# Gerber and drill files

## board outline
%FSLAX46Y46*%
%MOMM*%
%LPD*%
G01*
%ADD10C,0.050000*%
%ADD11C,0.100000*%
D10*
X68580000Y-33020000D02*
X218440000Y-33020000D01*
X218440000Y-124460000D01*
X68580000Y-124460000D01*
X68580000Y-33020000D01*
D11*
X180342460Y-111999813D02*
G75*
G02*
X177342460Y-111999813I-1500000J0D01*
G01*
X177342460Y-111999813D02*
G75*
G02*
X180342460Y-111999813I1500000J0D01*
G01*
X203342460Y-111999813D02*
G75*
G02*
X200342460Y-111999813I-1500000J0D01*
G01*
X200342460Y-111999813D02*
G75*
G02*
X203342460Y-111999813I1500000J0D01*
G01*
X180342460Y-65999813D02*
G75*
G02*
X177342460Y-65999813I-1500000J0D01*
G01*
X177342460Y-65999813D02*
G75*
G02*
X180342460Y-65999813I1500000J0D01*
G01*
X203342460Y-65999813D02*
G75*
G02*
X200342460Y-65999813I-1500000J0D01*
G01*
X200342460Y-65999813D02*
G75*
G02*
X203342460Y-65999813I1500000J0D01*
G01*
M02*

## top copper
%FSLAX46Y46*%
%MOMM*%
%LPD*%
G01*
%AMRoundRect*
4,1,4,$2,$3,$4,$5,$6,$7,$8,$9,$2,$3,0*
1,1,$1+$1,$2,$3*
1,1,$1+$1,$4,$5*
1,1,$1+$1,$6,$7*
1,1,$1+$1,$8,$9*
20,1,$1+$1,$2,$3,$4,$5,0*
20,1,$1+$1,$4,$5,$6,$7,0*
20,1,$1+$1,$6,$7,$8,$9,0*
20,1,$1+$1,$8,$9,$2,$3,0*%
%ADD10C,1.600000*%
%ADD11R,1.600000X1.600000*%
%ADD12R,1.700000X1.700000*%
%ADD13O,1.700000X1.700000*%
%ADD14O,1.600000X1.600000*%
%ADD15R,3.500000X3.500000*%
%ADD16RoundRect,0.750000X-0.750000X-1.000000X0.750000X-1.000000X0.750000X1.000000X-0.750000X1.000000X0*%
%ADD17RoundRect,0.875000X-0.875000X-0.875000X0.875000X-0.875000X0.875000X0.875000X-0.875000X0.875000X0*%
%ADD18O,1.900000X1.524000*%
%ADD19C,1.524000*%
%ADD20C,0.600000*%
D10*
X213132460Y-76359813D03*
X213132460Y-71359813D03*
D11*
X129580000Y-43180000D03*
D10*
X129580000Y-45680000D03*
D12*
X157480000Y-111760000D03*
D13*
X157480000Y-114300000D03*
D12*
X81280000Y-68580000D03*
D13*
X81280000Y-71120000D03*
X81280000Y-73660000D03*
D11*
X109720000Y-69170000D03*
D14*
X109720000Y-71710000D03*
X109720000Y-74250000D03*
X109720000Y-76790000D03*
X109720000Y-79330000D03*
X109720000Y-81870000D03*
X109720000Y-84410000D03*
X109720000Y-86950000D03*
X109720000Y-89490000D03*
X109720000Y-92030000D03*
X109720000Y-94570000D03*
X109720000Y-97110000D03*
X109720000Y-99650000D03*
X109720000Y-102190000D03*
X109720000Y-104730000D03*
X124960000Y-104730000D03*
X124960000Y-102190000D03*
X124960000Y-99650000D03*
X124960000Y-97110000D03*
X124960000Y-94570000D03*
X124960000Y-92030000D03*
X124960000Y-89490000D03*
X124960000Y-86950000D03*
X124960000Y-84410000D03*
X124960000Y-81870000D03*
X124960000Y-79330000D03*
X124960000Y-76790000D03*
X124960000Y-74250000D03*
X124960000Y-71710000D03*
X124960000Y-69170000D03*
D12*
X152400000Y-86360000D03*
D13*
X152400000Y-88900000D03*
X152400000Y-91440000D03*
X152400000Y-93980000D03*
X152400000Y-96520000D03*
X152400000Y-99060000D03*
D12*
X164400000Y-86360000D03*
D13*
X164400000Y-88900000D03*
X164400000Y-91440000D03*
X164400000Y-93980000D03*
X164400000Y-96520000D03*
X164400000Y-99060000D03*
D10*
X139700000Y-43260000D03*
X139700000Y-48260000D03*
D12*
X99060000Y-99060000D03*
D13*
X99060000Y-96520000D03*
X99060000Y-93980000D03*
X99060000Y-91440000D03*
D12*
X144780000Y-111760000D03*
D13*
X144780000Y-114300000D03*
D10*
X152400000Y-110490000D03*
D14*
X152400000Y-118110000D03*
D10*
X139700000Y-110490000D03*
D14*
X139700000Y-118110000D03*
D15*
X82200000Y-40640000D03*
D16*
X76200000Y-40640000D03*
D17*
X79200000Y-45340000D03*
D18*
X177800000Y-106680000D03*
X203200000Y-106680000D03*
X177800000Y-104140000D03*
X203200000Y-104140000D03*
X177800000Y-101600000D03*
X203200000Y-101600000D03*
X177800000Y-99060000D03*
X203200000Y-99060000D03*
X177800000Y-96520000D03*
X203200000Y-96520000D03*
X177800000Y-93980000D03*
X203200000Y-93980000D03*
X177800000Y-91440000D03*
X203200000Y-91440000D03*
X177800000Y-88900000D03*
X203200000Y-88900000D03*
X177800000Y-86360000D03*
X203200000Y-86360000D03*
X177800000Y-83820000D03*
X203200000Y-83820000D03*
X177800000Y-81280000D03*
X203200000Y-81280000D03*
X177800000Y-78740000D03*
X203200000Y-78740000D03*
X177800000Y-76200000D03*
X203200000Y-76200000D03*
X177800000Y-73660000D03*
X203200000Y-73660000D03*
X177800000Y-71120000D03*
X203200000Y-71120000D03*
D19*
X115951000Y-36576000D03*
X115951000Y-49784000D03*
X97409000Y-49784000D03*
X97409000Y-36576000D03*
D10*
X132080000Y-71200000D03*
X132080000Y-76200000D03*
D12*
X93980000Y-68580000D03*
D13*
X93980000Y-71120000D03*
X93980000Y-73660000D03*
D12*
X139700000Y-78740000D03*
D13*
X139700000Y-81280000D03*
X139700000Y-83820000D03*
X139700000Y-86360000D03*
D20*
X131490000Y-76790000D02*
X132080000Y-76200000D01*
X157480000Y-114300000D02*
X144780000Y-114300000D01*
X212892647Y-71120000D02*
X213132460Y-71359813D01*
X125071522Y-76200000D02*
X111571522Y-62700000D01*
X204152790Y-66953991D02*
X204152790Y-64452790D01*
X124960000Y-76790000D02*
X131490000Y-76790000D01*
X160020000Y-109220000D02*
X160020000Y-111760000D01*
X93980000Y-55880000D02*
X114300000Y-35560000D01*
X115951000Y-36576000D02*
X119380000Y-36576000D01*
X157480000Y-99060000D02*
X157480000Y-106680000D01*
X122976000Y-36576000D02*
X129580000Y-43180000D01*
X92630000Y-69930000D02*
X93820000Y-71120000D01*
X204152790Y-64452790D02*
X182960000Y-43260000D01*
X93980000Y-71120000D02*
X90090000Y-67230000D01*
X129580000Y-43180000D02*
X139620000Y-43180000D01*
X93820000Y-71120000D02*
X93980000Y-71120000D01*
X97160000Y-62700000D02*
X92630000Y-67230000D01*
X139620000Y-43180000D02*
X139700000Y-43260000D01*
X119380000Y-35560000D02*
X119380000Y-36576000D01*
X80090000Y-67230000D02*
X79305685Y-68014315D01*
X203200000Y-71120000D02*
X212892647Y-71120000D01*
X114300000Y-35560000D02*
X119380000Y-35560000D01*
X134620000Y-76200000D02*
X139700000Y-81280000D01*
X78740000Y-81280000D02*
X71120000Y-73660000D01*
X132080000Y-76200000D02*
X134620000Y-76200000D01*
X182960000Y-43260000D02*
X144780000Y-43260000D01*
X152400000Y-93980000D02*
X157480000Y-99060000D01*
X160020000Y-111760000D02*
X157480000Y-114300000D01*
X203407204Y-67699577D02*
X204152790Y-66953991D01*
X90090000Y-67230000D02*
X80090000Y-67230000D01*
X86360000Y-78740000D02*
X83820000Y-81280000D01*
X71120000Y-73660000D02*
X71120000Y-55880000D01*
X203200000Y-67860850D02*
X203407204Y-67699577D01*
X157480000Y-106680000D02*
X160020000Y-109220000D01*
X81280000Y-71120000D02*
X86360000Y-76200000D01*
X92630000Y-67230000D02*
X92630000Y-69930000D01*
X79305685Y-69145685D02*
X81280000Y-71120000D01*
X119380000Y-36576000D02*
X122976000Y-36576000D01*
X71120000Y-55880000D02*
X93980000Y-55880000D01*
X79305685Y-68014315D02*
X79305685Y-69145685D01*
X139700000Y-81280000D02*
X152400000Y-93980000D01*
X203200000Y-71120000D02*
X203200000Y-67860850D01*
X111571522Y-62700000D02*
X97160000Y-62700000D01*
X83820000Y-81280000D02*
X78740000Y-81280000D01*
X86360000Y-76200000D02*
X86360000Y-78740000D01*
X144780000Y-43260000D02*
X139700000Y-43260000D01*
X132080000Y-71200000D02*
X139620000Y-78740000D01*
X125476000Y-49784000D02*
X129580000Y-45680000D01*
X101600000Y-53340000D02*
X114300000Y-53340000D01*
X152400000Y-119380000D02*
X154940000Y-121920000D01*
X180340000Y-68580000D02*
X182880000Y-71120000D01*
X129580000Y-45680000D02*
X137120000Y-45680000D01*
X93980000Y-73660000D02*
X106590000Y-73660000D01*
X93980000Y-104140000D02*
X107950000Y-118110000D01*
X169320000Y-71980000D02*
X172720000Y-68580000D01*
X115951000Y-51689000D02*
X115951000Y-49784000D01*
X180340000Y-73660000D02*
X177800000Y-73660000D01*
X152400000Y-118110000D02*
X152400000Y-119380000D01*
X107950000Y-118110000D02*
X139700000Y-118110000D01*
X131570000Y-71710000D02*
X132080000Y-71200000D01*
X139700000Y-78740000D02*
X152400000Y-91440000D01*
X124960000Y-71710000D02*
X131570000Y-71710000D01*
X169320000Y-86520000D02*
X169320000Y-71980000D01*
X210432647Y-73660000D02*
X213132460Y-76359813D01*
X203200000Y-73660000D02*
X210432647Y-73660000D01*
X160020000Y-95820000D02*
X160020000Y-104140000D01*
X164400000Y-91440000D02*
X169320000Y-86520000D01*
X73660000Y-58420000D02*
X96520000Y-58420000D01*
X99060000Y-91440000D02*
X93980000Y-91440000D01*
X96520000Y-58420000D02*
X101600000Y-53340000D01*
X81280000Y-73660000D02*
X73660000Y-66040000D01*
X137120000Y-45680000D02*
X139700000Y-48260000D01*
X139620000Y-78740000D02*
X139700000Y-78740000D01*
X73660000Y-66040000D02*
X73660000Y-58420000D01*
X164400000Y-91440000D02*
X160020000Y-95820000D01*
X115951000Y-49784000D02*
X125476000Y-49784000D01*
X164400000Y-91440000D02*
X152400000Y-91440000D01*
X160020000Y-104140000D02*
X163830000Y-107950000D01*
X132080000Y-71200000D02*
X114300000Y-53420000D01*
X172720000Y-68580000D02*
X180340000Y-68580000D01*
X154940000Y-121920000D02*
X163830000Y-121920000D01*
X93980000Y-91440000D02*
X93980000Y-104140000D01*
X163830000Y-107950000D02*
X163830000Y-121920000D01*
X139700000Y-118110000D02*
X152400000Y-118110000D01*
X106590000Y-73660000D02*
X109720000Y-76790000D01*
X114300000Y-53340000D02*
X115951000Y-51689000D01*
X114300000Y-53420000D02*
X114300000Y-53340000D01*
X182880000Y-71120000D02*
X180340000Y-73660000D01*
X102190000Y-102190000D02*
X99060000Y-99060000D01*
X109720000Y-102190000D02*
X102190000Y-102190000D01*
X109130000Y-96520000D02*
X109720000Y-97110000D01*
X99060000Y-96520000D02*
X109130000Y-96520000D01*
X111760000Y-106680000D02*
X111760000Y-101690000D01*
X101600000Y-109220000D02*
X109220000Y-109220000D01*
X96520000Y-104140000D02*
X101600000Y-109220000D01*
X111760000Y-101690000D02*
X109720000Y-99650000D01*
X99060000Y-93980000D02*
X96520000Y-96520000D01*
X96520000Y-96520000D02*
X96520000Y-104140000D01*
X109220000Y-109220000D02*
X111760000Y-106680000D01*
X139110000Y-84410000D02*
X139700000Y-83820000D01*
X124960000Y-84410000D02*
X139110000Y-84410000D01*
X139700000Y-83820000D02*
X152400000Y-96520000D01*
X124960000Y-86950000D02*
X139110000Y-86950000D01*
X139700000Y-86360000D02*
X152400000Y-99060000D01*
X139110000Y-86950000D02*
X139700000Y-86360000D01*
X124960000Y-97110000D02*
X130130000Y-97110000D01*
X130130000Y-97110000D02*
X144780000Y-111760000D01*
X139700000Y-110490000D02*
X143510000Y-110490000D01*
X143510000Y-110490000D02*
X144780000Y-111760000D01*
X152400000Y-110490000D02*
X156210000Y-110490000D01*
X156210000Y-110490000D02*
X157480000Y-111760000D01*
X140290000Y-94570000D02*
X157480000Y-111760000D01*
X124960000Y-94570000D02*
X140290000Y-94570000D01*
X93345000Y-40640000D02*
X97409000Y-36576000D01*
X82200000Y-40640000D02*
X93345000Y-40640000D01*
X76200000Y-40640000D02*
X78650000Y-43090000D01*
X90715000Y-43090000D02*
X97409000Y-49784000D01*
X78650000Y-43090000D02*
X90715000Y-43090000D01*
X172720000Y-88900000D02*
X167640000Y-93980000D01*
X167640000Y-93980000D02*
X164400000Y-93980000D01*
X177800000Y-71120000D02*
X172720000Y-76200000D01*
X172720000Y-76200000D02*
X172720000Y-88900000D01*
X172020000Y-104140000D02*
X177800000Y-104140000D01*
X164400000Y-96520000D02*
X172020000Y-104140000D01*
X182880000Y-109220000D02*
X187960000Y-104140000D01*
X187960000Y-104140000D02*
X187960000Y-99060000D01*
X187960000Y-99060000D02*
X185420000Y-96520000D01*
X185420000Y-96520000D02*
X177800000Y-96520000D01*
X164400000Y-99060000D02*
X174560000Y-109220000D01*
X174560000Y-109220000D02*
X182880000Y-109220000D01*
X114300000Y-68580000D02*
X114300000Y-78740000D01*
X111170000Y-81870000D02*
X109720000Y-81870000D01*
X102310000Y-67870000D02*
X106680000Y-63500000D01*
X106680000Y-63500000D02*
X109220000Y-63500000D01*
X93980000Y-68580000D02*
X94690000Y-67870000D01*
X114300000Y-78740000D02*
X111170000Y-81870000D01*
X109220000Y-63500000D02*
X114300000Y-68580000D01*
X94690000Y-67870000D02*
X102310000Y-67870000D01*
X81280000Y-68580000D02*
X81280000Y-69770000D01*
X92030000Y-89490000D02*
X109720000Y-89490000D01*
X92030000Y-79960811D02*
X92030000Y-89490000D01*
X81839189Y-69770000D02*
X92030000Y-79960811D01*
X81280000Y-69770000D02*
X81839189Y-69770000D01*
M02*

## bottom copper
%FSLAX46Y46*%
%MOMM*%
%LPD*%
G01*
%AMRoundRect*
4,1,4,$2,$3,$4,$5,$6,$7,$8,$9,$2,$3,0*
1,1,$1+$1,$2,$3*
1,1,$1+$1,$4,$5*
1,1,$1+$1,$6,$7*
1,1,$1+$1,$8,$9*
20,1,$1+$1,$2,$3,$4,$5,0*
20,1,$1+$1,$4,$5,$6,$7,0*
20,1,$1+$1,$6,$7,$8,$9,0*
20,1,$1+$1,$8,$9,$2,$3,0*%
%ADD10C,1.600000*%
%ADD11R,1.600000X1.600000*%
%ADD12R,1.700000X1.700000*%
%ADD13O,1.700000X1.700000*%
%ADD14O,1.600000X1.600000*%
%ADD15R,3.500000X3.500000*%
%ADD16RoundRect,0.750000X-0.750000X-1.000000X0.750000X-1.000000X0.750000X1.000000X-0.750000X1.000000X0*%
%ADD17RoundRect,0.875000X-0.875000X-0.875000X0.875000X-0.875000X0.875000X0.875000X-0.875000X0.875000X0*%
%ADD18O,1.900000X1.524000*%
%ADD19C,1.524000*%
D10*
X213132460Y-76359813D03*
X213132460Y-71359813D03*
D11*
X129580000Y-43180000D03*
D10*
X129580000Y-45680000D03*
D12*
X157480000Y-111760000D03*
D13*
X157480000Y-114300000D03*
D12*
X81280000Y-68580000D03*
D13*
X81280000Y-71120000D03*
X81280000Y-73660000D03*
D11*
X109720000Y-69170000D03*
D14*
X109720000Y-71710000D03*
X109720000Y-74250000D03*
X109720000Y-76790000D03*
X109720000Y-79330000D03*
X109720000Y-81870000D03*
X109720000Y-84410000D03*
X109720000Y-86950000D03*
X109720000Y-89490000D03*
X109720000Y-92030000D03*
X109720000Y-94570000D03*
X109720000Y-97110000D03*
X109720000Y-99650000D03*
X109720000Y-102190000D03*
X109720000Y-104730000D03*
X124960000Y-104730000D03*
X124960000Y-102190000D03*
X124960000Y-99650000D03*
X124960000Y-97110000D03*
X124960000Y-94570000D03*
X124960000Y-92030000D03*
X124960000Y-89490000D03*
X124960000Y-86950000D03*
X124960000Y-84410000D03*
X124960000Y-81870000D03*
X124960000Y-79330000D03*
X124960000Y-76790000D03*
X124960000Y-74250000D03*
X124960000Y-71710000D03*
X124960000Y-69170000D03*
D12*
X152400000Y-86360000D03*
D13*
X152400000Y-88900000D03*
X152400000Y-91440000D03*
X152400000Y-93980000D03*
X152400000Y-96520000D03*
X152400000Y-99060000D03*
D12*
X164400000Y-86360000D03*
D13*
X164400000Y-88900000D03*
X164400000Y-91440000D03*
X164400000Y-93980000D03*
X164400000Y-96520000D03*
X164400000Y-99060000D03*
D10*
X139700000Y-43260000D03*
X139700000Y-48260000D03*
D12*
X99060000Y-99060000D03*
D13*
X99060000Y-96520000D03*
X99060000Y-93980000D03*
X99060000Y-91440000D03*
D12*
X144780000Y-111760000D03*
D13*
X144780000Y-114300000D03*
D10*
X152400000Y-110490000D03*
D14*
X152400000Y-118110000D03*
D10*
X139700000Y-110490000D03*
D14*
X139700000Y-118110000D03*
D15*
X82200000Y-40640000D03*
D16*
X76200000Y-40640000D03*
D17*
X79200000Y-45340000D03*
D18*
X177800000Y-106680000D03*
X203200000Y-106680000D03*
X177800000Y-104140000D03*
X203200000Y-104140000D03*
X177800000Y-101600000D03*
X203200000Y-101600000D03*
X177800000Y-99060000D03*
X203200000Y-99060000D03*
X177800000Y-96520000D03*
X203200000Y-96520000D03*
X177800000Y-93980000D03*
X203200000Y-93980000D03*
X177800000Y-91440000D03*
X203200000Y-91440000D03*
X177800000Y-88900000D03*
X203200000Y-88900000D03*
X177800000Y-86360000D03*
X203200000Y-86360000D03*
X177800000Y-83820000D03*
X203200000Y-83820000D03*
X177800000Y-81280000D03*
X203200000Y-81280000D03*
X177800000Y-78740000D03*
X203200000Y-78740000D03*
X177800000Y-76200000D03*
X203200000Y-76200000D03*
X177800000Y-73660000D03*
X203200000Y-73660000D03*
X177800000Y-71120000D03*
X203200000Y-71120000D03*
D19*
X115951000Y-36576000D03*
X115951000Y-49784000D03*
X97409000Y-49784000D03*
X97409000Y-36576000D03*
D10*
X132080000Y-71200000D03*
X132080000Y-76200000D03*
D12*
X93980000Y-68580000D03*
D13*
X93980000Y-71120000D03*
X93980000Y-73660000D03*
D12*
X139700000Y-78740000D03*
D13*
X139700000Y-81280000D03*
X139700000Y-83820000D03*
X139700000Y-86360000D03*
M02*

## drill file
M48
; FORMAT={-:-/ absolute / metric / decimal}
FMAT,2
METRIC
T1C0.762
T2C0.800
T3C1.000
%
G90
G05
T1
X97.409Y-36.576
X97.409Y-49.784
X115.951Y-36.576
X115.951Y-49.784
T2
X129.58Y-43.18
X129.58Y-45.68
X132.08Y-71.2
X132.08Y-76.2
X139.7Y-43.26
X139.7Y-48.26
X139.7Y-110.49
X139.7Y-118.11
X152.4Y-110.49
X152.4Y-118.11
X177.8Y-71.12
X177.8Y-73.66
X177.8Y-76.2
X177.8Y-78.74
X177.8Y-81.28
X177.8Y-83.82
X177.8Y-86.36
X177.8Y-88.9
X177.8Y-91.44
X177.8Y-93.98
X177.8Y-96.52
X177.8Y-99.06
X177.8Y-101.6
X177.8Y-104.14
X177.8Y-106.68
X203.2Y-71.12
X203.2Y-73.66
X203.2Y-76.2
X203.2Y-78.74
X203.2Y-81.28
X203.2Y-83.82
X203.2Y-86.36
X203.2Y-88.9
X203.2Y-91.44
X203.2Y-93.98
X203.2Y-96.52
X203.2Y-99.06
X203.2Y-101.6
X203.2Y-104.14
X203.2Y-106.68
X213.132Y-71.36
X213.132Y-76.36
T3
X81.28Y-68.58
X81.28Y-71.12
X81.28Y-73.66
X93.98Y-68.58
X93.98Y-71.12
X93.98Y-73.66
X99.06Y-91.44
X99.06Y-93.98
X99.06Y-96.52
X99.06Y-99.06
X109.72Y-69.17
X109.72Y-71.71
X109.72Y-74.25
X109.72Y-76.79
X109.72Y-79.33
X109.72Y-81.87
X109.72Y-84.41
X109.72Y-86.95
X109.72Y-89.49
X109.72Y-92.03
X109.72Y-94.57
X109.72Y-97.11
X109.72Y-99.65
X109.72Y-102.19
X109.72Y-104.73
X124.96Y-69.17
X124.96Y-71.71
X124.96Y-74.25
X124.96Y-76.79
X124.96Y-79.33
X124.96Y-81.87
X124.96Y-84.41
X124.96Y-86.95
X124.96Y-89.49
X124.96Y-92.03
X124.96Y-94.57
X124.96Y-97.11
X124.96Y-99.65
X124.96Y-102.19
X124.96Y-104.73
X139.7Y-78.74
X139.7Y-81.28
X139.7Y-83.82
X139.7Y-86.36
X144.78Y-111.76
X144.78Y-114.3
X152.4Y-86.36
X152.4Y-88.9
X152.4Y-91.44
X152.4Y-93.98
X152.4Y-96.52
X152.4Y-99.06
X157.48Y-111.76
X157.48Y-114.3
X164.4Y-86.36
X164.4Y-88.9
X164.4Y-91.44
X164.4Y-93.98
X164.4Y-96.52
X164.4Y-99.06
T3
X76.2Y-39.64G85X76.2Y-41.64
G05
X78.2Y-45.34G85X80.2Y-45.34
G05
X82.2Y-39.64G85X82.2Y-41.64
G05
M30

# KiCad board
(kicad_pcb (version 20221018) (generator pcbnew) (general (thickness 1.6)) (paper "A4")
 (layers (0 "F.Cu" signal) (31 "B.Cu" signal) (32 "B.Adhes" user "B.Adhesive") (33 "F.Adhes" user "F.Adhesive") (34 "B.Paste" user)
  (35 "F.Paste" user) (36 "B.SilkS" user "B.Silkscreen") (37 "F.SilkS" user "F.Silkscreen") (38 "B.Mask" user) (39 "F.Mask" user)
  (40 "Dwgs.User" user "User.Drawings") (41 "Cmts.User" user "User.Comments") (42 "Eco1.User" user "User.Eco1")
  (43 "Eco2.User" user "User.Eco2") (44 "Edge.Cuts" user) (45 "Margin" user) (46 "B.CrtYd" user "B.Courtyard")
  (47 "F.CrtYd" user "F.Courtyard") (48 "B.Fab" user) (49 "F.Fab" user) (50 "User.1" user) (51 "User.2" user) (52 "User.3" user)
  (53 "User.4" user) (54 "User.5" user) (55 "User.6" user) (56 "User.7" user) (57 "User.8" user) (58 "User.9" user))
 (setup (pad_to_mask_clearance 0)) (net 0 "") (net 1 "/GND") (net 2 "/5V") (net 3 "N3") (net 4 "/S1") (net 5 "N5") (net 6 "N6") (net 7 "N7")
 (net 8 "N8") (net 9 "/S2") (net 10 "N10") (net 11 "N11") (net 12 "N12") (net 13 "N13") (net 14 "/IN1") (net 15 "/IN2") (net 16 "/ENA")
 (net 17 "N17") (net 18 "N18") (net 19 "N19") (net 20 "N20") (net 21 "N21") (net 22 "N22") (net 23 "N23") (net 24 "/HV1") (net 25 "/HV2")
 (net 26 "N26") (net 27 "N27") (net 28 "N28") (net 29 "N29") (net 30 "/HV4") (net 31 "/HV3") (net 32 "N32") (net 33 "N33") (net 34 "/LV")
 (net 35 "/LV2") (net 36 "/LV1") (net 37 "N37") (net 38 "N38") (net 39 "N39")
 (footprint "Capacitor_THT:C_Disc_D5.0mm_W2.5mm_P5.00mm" (layer "F.Cu") (at 213.13246 76.359813 90)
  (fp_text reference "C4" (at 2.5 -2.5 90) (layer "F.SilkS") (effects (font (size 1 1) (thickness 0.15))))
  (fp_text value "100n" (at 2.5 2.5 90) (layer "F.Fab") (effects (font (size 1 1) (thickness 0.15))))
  (pad "1" thru_hole circle (at 0 0 90) (size 1.6 1.6) (drill 0.8) (layers "*.Cu" "*.Mask") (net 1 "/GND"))
  (pad "2" thru_hole circle (at 5 0 90) (size 1.6 1.6) (drill 0.8) (layers "*.Cu" "*.Mask") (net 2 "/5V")))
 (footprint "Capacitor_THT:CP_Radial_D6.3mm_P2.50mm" (layer "F.Cu") (at 129.58 43.18 -90)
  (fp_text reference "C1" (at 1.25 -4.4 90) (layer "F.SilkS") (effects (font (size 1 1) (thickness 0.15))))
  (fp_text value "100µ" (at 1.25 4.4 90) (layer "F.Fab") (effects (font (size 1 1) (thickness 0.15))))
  (pad "1" thru_hole rect (at 0 0 270) (size 1.6 1.6) (drill 0.8) (layers "*.Cu" "*.Mask") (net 2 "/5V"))
  (pad "2" thru_hole circle (at 2.5 0 270) (size 1.6 1.6) (drill 0.8) (layers "*.Cu" "*.Mask") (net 1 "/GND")))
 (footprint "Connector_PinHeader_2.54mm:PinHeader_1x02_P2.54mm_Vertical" (layer "F.Cu") (at 157.48 111.76)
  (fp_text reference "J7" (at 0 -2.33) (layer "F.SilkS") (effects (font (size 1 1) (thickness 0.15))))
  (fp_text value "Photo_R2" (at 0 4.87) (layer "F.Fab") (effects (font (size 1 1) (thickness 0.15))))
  (pad "1" thru_hole rect (at 0 0) (size 1.7 1.7) (drill 1) (layers "*.Cu" "*.Mask") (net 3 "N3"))
  (pad "2" thru_hole oval (at 0 2.54) (size 1.7 1.7) (drill 1) (layers "*.Cu" "*.Mask") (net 2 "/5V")))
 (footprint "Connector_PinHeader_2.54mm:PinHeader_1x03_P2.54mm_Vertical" (layer "F.Cu") (at 81.28 68.58)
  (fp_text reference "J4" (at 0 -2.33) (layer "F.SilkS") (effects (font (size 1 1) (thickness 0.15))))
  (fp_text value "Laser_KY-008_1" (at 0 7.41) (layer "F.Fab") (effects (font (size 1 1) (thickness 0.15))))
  (pad "1" thru_hole rect (at 0 0) (size 1.7 1.7) (drill 1) (layers "*.Cu" "*.Mask") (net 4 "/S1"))
  (pad "2" thru_hole oval (at 0 2.54) (size 1.7 1.7) (drill 1) (layers "*.Cu" "*.Mask") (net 2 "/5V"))
  (pad "3" thru_hole oval (at 0 5.08) (size 1.7 1.7) (drill 1) (layers "*.Cu" "*.Mask") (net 1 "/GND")))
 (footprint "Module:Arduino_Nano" (layer "F.Cu") (at 109.72 69.17)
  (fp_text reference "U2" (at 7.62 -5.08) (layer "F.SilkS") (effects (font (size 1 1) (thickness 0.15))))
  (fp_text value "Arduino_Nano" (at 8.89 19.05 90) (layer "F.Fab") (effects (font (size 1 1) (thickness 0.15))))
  (pad "1" thru_hole rect (at 0 0) (size 1.6 1.6) (drill 1) (layers "*.Cu" "*.Mask") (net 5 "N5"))
  (pad "2" thru_hole oval (at 0 2.54) (size 1.6 1.6) (drill 1) (layers "*.Cu" "*.Mask") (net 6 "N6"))
  (pad "3" thru_hole oval (at 0 5.08) (size 1.6 1.6) (drill 1) (layers "*.Cu" "*.Mask") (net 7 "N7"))
  (pad "4" thru_hole oval (at 0 7.62) (size 1.6 1.6) (drill 1) (layers "*.Cu" "*.Mask") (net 1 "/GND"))
  (pad "5" thru_hole oval (at 0 10.16) (size 1.6 1.6) (drill 1) (layers "*.Cu" "*.Mask") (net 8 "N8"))
  (pad "6" thru_hole oval (at 0 12.7) (size 1.6 1.6) (drill 1) (layers "*.Cu" "*.Mask") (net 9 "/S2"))
  (pad "7" thru_hole oval (at 0 15.24) (size 1.6 1.6) (drill 1) (layers "*.Cu" "*.Mask") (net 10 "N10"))
  (pad "8" thru_hole oval (at 0 17.78) (size 1.6 1.6) (drill 1) (layers "*.Cu" "*.Mask") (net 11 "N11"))
  (pad "9" thru_hole oval (at 0 20.32) (size 1.6 1.6) (drill 1) (layers "*.Cu" "*.Mask") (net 4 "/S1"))
  (pad "10" thru_hole oval (at 0 22.86) (size 1.6 1.6) (drill 1) (layers "*.Cu" "*.Mask") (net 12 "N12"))
  (pad "11" thru_hole oval (at 0 25.4) (size 1.6 1.6) (drill 1) (layers "*.Cu" "*.Mask") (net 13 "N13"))
  (pad "12" thru_hole oval (at 0 27.94) (size 1.6 1.6) (drill 1) (layers "*.Cu" "*.Mask") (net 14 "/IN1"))
  (pad "13" thru_hole oval (at 0 30.48) (size 1.6 1.6) (drill 1) (layers "*.Cu" "*.Mask") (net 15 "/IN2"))
  (pad "14" thru_hole oval (at 0 33.02) (size 1.6 1.6) (drill 1) (layers "*.Cu" "*.Mask") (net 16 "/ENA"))
  (pad "15" thru_hole oval (at 0 35.56) (size 1.6 1.6) (drill 1) (layers "*.Cu" "*.Mask") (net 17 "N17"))
  (pad "16" thru_hole oval (at 15.24 35.56) (size 1.6 1.6) (drill 1) (layers "*.Cu" "*.Mask") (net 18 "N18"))
  (pad "17" thru_hole oval (at 15.24 33.02) (size 1.6 1.6) (drill 1) (layers "*.Cu" "*.Mask") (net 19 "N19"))
  (pad "18" thru_hole oval (at 15.24 30.48) (size 1.6 1.6) (drill 1) (layers "*.Cu" "*.Mask") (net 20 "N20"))
  (pad "19" thru_hole oval (at 15.24 27.94) (size 1.6 1.6) (drill 1) (layers "*.Cu" "*.Mask") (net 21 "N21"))
  (pad "20" thru_hole oval (at 15.24 25.4) (size 1.6 1.6) (drill 1) (layers "*.Cu" "*.Mask") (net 3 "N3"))
  (pad "21" thru_hole oval (at 15.24 22.86) (size 1.6 1.6) (drill 1) (layers "*.Cu" "*.Mask") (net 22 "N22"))
  (pad "22" thru_hole oval (at 15.24 20.32) (size 1.6 1.6) (drill 1) (layers "*.Cu" "*.Mask") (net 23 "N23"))
  (pad "23" thru_hole oval (at 15.24 17.78) (size 1.6 1.6) (drill 1) (layers "*.Cu" "*.Mask") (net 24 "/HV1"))
  (pad "24" thru_hole oval (at 15.24 15.24) (size 1.6 1.6) (drill 1) (layers "*.Cu" "*.Mask") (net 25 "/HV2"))
  (pad "25" thru_hole oval (at 15.24 12.7) (size 1.6 1.6) (drill 1) (layers "*.Cu" "*.Mask") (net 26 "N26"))
  (pad "26" thru_hole oval (at 15.24 10.16) (size 1.6 1.6) (drill 1) (layers "*.Cu" "*.Mask") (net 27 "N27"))
  (pad "27" thru_hole oval (at 15.24 7.62) (size 1.6 1.6) (drill 1) (layers "*.Cu" "*.Mask") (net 2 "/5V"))
  (pad "28" thru_hole oval (at 15.24 5.08) (size 1.6 1.6) (drill 1) (layers "*.Cu" "*.Mask") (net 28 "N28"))
  (pad "29" thru_hole oval (at 15.24 2.54) (size 1.6 1.6) (drill 1) (layers "*.Cu" "*.Mask") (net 1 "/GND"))
  (pad "30" thru_hole oval (at 15.24 0) (size 1.6 1.6) (drill 1) (layers "*.Cu" "*.Mask") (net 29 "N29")))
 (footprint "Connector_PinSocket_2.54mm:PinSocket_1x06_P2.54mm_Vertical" (layer "F.Cu") (at 152.4 86.36)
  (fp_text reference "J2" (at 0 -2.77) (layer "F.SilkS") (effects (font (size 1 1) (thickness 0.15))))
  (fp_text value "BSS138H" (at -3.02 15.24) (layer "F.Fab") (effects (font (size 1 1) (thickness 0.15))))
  (pad "1" thru_hole rect (at 0 0) (size 1.7 1.7) (drill 1) (layers "*.Cu" "*.Mask") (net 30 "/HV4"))
  (pad "2" thru_hole oval (at 0 2.54) (size 1.7 1.7) (drill 1) (layers "*.Cu" "*.Mask") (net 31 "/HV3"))
  (pad "3" thru_hole oval (at 0 5.08) (size 1.7 1.7) (drill 1) (layers "*.Cu" "*.Mask") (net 1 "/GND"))
  (pad "4" thru_hole oval (at 0 7.62) (size 1.7 1.7) (drill 1) (layers "*.Cu" "*.Mask") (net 2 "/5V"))
  (pad "5" thru_hole oval (at 0 10.16) (size 1.7 1.7) (drill 1) (layers "*.Cu" "*.Mask") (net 25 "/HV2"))
  (pad "6" thru_hole oval (at 0 12.7) (size 1.7 1.7) (drill 1) (layers "*.Cu" "*.Mask") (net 24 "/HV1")))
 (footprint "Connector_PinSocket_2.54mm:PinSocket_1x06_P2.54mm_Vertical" (layer "F.Cu") (at 164.4 86.36)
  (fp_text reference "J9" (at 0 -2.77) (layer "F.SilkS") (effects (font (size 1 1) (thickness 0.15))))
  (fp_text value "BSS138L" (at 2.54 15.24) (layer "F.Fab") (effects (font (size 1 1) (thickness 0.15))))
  (pad "1" thru_hole rect (at 0 0) (size 1.7 1.7) (drill 1) (layers "*.Cu" "*.Mask") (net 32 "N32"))
  (pad "2" thru_hole oval (at 0 2.54) (size 1.7 1.7) (drill 1) (layers "*.Cu" "*.Mask") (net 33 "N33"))
  (pad "3" thru_hole oval (at 0 5.08) (size 1.7 1.7) (drill 1) (layers "*.Cu" "*.Mask") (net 1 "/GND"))
  (pad "4" thru_hole oval (at 0 7.62) (size 1.7 1.7) (drill 1) (layers "*.Cu" "*.Mask") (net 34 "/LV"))
  (pad "5" thru_hole oval (at 0 10.16) (size 1.7 1.7) (drill 1) (layers "*.Cu" "*.Mask") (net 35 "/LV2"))
  (pad "6" thru_hole oval (at 0 12.7) (size 1.7 1.7) (drill 1) (layers "*.Cu" "*.Mask") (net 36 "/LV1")))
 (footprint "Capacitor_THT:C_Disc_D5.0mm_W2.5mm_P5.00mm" (layer "F.Cu") (at 139.7 43.26 -90)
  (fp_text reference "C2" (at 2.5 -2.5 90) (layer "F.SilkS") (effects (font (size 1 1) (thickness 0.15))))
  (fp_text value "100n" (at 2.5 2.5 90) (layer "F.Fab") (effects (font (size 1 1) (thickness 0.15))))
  (pad "1" thru_hole circle (at 0 0 270) (size 1.6 1.6) (drill 0.8) (layers "*.Cu" "*.Mask") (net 2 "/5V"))
  (pad "2" thru_hole circle (at 5 0 270) (size 1.6 1.6) (drill 0.8) (layers "*.Cu" "*.Mask") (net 1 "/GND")))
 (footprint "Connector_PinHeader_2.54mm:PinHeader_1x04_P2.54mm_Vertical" (layer "F.Cu") (at 99.06 99.06 180)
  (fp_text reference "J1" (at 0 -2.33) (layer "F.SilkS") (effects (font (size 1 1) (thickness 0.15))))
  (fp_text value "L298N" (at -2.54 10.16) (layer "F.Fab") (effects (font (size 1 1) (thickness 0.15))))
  (pad "1" thru_hole rect (at 0 0 180) (size 1.7 1.7) (drill 1) (layers "*.Cu" "*.Mask") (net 16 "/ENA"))
  (pad "2" thru_hole oval (at 0 2.54 180) (size 1.7 1.7) (drill 1) (layers "*.Cu" "*.Mask") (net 14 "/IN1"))
  (pad "3" thru_hole oval (at 0 5.08 180) (size 1.7 1.7) (drill 1) (layers "*.Cu" "*.Mask") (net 15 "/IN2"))
  (pad "4" thru_hole oval (at 0 7.62 180) (size 1.7 1.7) (drill 1) (layers "*.Cu" "*.Mask") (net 1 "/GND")))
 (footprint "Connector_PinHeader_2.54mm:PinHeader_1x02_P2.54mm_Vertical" (layer "F.Cu") (at 144.78 111.76)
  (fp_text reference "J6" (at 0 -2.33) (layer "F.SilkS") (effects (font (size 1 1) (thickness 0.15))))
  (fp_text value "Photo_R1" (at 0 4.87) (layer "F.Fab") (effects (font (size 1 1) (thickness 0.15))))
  (pad "1" thru_hole rect (at 0 0) (size 1.7 1.7) (drill 1) (layers "*.Cu" "*.Mask") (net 21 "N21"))
  (pad "2" thru_hole oval (at 0 2.54) (size 1.7 1.7) (drill 1) (layers "*.Cu" "*.Mask") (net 2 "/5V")))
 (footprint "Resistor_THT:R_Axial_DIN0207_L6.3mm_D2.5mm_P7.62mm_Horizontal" (layer "F.Cu") (at 152.4 110.49 -90)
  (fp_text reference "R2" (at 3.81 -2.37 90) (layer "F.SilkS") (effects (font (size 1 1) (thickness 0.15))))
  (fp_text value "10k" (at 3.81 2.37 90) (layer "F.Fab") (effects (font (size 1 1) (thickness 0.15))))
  (pad "1" thru_hole circle (at 0 0 270) (size 1.6 1.6) (drill 0.8) (layers "*.Cu" "*.Mask") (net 3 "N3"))
  (pad "2" thru_hole oval (at 7.62 0 270) (size 1.6 1.6) (drill 0.8) (layers "*.Cu" "*.Mask") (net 1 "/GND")))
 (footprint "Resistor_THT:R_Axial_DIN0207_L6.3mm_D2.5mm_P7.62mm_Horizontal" (layer "F.Cu") (at 139.7 110.49 -90)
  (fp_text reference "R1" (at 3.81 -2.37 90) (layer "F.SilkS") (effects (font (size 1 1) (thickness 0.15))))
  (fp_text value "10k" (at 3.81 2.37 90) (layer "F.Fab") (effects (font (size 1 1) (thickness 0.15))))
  (pad "1" thru_hole circle (at 0 0 270) (size 1.6 1.6) (drill 0.8) (layers "*.Cu" "*.Mask") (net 21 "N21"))
  (pad "2" thru_hole oval (at 7.62 0 270) (size 1.6 1.6) (drill 0.8) (layers "*.Cu" "*.Mask") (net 1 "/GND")))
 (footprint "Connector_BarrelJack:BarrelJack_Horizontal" (layer "F.Cu") (at 82.2 40.64)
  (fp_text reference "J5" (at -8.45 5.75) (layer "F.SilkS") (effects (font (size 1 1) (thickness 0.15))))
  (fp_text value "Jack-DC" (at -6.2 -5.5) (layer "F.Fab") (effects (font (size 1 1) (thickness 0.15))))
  (pad "1" thru_hole rect (at 0 0) (size 3.5 3.5) (drill oval 1 3) (layers "*.Cu" "*.Mask") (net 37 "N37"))
  (pad "2" thru_hole roundrect (at -6 0) (size 3 3.5) (drill oval 1 3) (layers "*.Cu" "*.Mask") (roundrect_rratio 0.25) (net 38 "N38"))
  (pad "3" thru_hole roundrect (at -3 4.7) (size 3.5 3.5) (drill oval 3 1) (layers "*.Cu" "*.Mask") (roundrect_rratio 0.25)))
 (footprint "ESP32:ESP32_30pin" (layer "F.Cu") (at 190.27246 89.139813 90)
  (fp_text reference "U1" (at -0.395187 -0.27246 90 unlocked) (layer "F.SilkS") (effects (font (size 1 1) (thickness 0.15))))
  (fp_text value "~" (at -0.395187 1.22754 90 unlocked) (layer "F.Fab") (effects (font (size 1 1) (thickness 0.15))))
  (fp_circle (center -22.86 -11.43) (end -21.36 -11.43) (stroke (width 0.1) (type default)) (fill none) (layer "Edge.Cuts"))
  (fp_circle (center -22.86 11.57) (end -21.36 11.57) (stroke (width 0.1) (type default)) (fill none) (layer "Edge.Cuts"))
  (fp_circle (center 23.14 -11.43) (end 24.64 -11.43) (stroke (width 0.1) (type default)) (fill none) (layer "Edge.Cuts"))
  (fp_circle (center 23.14 11.57) (end 24.64 11.57) (stroke (width 0.1) (type default)) (fill none) (layer "Edge.Cuts"))
  (pad "1" thru_hole oval (at -17.540187 -12.47246 90) (size 1.524 1.9) (drill 0.8) (layers "*.Cu" "*.Mask"))
  (pad "1" thru_hole oval (at -17.540187 12.92754 90) (size 1.524 1.9) (drill 0.8) (layers "*.Cu" "*.Mask"))
  (pad "2" thru_hole oval (at -15.000187 -12.47246 90) (size 1.524 1.9) (drill 0.8) (layers "*.Cu" "*.Mask") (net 35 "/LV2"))
  (pad "2" thru_hole oval (at -15.000187 12.92754 90) (size 1.524 1.9) (drill 0.8) (layers "*.Cu" "*.Mask"))
  (pad "3" thru_hole oval (at -12.460187 -12.47246 90) (size 1.524 1.9) (drill 0.8) (layers "*.Cu" "*.Mask") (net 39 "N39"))
  (pad "3" thru_hole oval (at -12.460187 12.92754 90) (size 1.524 1.9) (drill 0.8) (layers "*.Cu" "*.Mask"))
  (pad "4" thru_hole oval (at -9.920187 -12.47246 90) (size 1.524 1.9) (drill 0.8) (layers "*.Cu" "*.Mask"))
  (pad "4" thru_hole oval (at -9.920187 12.92754 90) (size 1.524 1.9) (drill 0.8) (layers "*.Cu" "*.Mask"))
  (pad "5" thru_hole oval (at -7.380187 -12.47246 90) (size 1.524 1.9) (drill 0.8) (layers "*.Cu" "*.Mask") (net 36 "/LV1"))
  (pad "5" thru_hole oval (at -7.380187 12.92754 90) (size 1.524 1.9) (drill 0.8) (layers "*.Cu" "*.Mask"))
  (pad "6" thru_hole oval (at -4.840187 -12.47246 90) (size 1.524 1.9) (drill 0.8) (layers "*.Cu" "*.Mask"))
  (pad "6" thru_hole oval (at -4.840187 12.92754 90) (size 1.524 1.9) (drill 0.8) (layers "*.Cu" "*.Mask"))
  (pad "7" thru_hole oval (at -2.300187 -12.47246 90) (size 1.524 1.9) (drill 0.8) (layers "*.Cu" "*.Mask"))
  (pad "7" thru_hole oval (at -2.300187 12.92754 90) (size 1.524 1.9) (drill 0.8) (layers "*.Cu" "*.Mask"))
  (pad "8" thru_hole oval (at 0.239813 -12.47246 90) (size 1.524 1.9) (drill 0.8) (layers "*.Cu" "*.Mask"))
  (pad "8" thru_hole oval (at 0.239813 12.92754 90) (size 1.524 1.9) (drill 0.8) (layers "*.Cu" "*.Mask"))
  (pad "9" thru_hole oval (at 2.779813 -12.47246 90) (size 1.524 1.9) (drill 0.8) (layers "*.Cu" "*.Mask"))
  (pad "9" thru_hole oval (at 2.779813 12.92754 90) (size 1.524 1.9) (drill 0.8) (layers "*.Cu" "*.Mask"))
  (pad "10" thru_hole oval (at 5.319813 -12.47246 90) (size 1.524 1.9) (drill 0.8) (layers "*.Cu" "*.Mask"))
  (pad "10" thru_hole oval (at 5.319813 12.92754 90) (size 1.524 1.9) (drill 0.8) (layers "*.Cu" "*.Mask"))
  (pad "11" thru_hole oval (at 7.859813 -12.47246 90) (size 1.524 1.9) (drill 0.8) (layers "*.Cu" "*.Mask"))
  (pad "11" thru_hole oval (at 7.859813 12.92754 90) (size 1.524 1.9) (drill 0.8) (layers "*.Cu" "*.Mask"))
  (pad "12" thru_hole oval (at 10.399813 -12.47246 90) (size 1.524 1.9) (drill 0.8) (layers "*.Cu" "*.Mask"))
  (pad "12" thru_hole oval (at 10.399813 12.92754 90) (size 1.524 1.9) (drill 0.8) (layers "*.Cu" "*.Mask"))
  (pad "13" thru_hole oval (at 12.939813 -12.47246 90) (size 1.524 1.9) (drill 0.8) (layers "*.Cu" "*.Mask"))
  (pad "13" thru_hole oval (at 12.939813 12.92754 90) (size 1.524 1.9) (drill 0.8) (layers "*.Cu" "*.Mask"))
  (pad "14" thru_hole oval (at 15.479813 -12.47246 90) (size 1.524 1.9) (drill 0.8) (layers "*.Cu" "*.Mask") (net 1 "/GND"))
  (pad "14" thru_hole oval (at 15.479813 12.92754 90) (size 1.524 1.9) (drill 0.8) (layers "*.Cu" "*.Mask") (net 1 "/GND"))
  (pad "15" thru_hole oval (at 18.019813 -12.47246 90) (size 1.524 1.9) (drill 0.8) (layers "*.Cu" "*.Mask") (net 34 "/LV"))
  (pad "15" thru_hole oval (at 18.019813 12.92754 90) (size 1.524 1.9) (drill 0.8) (layers "*.Cu" "*.Mask") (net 2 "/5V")))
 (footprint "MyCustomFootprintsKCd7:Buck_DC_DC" (layer "F.Cu") (at 106.68 43.18)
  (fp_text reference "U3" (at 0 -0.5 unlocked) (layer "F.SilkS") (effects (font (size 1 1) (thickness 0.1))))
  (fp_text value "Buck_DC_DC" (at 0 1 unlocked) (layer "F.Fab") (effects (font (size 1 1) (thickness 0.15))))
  (pad "1" thru_hole circle (at 9.271 -6.604) (size 1.524 1.524) (drill 0.762) (layers "*.Cu" "*.Mask") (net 2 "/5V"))
  (pad "2" thru_hole circle (at 9.271 6.604) (size 1.524 1.524) (drill 0.762) (layers "*.Cu" "*.Mask") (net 1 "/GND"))
  (pad "3" thru_hole circle (at -9.271 6.604) (size 1.524 1.524) (drill 0.762) (layers "*.Cu" "*.Mask") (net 38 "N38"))
  (pad "4" thru_hole circle (at -9.271 -6.604) (size 1.524 1.524) (drill 0.762) (layers "*.Cu" "*.Mask") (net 37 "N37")))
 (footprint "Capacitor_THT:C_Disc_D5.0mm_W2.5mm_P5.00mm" (layer "F.Cu") (at 132.08 71.2 -90)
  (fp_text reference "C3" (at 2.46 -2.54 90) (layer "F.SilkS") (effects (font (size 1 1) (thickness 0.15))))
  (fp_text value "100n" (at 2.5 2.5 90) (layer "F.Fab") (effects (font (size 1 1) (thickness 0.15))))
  (pad "1" thru_hole circle (at 0 0 270) (size 1.6 1.6) (drill 0.8) (layers "*.Cu" "*.Mask") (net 1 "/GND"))
  (pad "2" thru_hole circle (at 5 0 270) (size 1.6 1.6) (drill 0.8) (layers "*.Cu" "*.Mask") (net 2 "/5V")))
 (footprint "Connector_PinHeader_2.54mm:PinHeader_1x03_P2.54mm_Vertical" (layer "F.Cu") (at 93.98 68.58)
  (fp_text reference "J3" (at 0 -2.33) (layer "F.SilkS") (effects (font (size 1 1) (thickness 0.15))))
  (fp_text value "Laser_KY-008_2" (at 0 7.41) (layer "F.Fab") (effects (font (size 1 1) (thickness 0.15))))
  (pad "1" thru_hole rect (at 0 0) (size 1.7 1.7) (drill 1) (layers "*.Cu" "*.Mask") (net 9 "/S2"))
  (pad "2" thru_hole oval (at 0 2.54) (size 1.7 1.7) (drill 1) (layers "*.Cu" "*.Mask") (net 2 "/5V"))
  (pad "3" thru_hole oval (at 0 5.08) (size 1.7 1.7) (drill 1) (layers "*.Cu" "*.Mask") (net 1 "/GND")))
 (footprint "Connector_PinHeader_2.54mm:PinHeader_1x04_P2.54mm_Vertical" (layer "F.Cu") (at 139.7 78.74)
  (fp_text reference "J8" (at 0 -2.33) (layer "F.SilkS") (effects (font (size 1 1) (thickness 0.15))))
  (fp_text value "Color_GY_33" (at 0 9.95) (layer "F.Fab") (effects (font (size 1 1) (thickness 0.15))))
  (pad "1" thru_hole rect (at 0 0) (size 1.7 1.7) (drill 1) (layers "*.Cu" "*.Mask") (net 1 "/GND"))
  (pad "2" thru_hole oval (at 0 2.54) (size 1.7 1.7) (drill 1) (layers "*.Cu" "*.Mask") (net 2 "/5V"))
  (pad "3" thru_hole oval (at 0 5.08) (size 1.7 1.7) (drill 1) (layers "*.Cu" "*.Mask") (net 25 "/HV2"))
  (pad "4" thru_hole oval (at 0 7.62) (size 1.7 1.7) (drill 1) (layers "*.Cu" "*.Mask") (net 24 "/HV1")))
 (gr_rect (start 68.58 33.02) (end 218.44 124.46) (stroke (width 0.05) (type default)) (fill none) (layer "Edge.Cuts"))
 (segment (start 131.49 76.79) (end 132.08 76.2) (width 0.6) (layer "F.Cu") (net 2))
 (segment (start 157.48 114.3) (end 144.78 114.3) (width 0.6) (layer "F.Cu") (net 2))
 (segment (start 212.892647 71.12) (end 213.13246 71.359813) (width 0.6) (layer "F.Cu") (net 2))
 (segment (start 125.071522 76.2) (end 111.571522 62.7) (width 0.6) (layer "F.Cu") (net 2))
 (segment (start 204.15279 66.953991) (end 204.15279 64.45279) (width 0.6) (layer "F.Cu") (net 2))
 (segment (start 124.96 76.79) (end 131.49 76.79) (width 0.6) (layer "F.Cu") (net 2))
 (segment (start 160.02 109.22) (end 160.02 111.76) (width 0.6) (layer "F.Cu") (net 2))
 (segment (start 93.98 55.88) (end 114.3 35.56) (width 0.6) (layer "F.Cu") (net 2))
 (segment (start 115.951 36.576) (end 119.38 36.576) (width 0.6) (layer "F.Cu") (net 2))
 (segment (start 157.48 99.06) (end 157.48 106.68) (width 0.6) (layer "F.Cu") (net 2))
 (segment (start 122.976 36.576) (end 129.58 43.18) (width 0.6) (layer "F.Cu") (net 2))
 (segment (start 92.63 69.93) (end 93.82 71.12) (width 0.6) (layer "F.Cu") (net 2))
 (segment (start 204.15279 64.45279) (end 182.96 43.26) (width 0.6) (layer "F.Cu") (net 2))
 (segment (start 93.98 71.12) (end 90.09 67.23) (width 0.6) (layer "F.Cu") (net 2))
 (segment (start 129.58 43.18) (end 139.62 43.18) (width 0.6) (layer "F.Cu") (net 2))
 (segment (start 93.82 71.12) (end 93.98 71.12) (width 0.6) (layer "F.Cu") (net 2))
 (segment (start 97.16 62.7) (end 92.63 67.23) (width 0.6) (layer "F.Cu") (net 2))
 (segment (start 139.62 43.18) (end 139.7 43.26) (width 0.6) (layer "F.Cu") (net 2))
 (segment (start 119.38 35.56) (end 119.38 36.576) (width 0.6) (layer "F.Cu") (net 2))
 (segment (start 80.09 67.23) (end 79.305685 68.014315) (width 0.6) (layer "F.Cu") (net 2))
 (segment (start 203.2 71.12) (end 212.892647 71.12) (width 0.6) (layer "F.Cu") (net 2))
 (segment (start 114.3 35.56) (end 119.38 35.56) (width 0.6) (layer "F.Cu") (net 2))
 (segment (start 134.62 76.2) (end 139.7 81.28) (width 0.6) (layer "F.Cu") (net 2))
 (segment (start 78.74 81.28) (end 71.12 73.66) (width 0.6) (layer "F.Cu") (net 2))
 (segment (start 132.08 76.2) (end 134.62 76.2) (width 0.6) (layer "F.Cu") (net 2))
 (segment (start 182.96 43.26) (end 144.78 43.26) (width 0.6) (layer "F.Cu") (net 2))
 (segment (start 152.4 93.98) (end 157.48 99.06) (width 0.6) (layer "F.Cu") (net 2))
 (segment (start 160.02 111.76) (end 157.48 114.3) (width 0.6) (layer "F.Cu") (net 2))
 (segment (start 203.407204 67.699577) (end 204.15279 66.953991) (width 0.6) (layer "F.Cu") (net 2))
 (segment (start 90.09 67.23) (end 80.09 67.23) (width 0.6) (layer "F.Cu") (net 2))
 (segment (start 86.36 78.74) (end 83.82 81.28) (width 0.6) (layer "F.Cu") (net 2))
 (segment (start 71.12 73.66) (end 71.12 55.88) (width 0.6) (layer "F.Cu") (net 2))
 (segment (start 203.2 67.86085) (end 203.407204 67.699577) (width 0.6) (layer "F.Cu") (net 2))
 (segment (start 157.48 106.68) (end 160.02 109.22) (width 0.6) (layer "F.Cu") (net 2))
 (segment (start 81.28 71.12) (end 86.36 76.2) (width 0.6) (layer "F.Cu") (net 2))
 (segment (start 92.63 67.23) (end 92.63 69.93) (width 0.6) (layer "F.Cu") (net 2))
 (segment (start 79.305685 69.145685) (end 81.28 71.12) (width 0.6) (layer "F.Cu") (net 2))
 (segment (start 119.38 36.576) (end 122.976 36.576) (width 0.6) (layer "F.Cu") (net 2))
 (segment (start 71.12 55.88) (end 93.98 55.88) (width 0.6) (layer "F.Cu") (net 2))
 (segment (start 79.305685 68.014315) (end 79.305685 69.145685) (width 0.6) (layer "F.Cu") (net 2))
 (segment (start 139.7 81.28) (end 152.4 93.98) (width 0.6) (layer "F.Cu") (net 2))
 (segment (start 203.2 71.12) (end 203.2 67.86085) (width 0.6) (layer "F.Cu") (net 2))
 (segment (start 111.571522 62.7) (end 97.16 62.7) (width 0.6) (layer "F.Cu") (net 2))
 (segment (start 83.82 81.28) (end 78.74 81.28) (width 0.6) (layer "F.Cu") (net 2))
 (segment (start 86.36 76.2) (end 86.36 78.74) (width 0.6) (layer "F.Cu") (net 2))
 (segment (start 144.78 43.26) (end 139.7 43.26) (width 0.6) (layer "F.Cu") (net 2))
 (segment (start 132.08 71.2) (end 139.62 78.74) (width 0.6) (layer "F.Cu") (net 1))
 (segment (start 125.476 49.784) (end 129.58 45.68) (width 0.6) (layer "F.Cu") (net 1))
 (segment (start 101.6 53.34) (end 114.3 53.34) (width 0.6) (layer "F.Cu") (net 1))
 (segment (start 152.4 119.38) (end 154.94 121.92) (width 0.6) (layer "F.Cu") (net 1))
 (segment (start 180.34 68.58) (end 182.88 71.12) (width 0.6) (layer "F.Cu") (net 1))
 (segment (start 129.58 45.68) (end 137.12 45.68) (width 0.6) (layer "F.Cu") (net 1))
 (segment (start 93.98 73.66) (end 106.59 73.66) (width 0.6) (layer "F.Cu") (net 1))
 (segment (start 93.98 104.14) (end 107.95 118.11) (width 0.6) (layer "F.Cu") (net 1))
 (segment (start 169.32 71.98) (end 172.72 68.58) (width 0.6) (layer "F.Cu") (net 1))
 (segment (start 115.951 51.689) (end 115.951 49.784) (width 0.6) (layer "F.Cu") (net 1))
 (segment (start 180.34 73.66) (end 177.8 73.66) (width 0.6) (layer "F.Cu") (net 1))
 (segment (start 152.4 118.11) (end 152.4 119.38) (width 0.6) (layer "F.Cu") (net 1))
 (segment (start 107.95 118.11) (end 139.7 118.11) (width 0.6) (layer "F.Cu") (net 1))
 (segment (start 131.57 71.71) (end 132.08 71.2) (width 0.6) (layer "F.Cu") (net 1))
 (segment (start 139.7 78.74) (end 152.4 91.44) (width 0.6) (layer "F.Cu") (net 1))
 (segment (start 124.96 71.71) (end 131.57 71.71) (width 0.6) (layer "F.Cu") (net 1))
 (segment (start 169.32 86.52) (end 169.32 71.98) (width 0.6) (layer "F.Cu") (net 1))
 (segment (start 210.432647 73.66) (end 213.13246 76.359813) (width 0.6) (layer "F.Cu") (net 1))
 (segment (start 203.2 73.66) (end 210.432647 73.66) (width 0.6) (layer "F.Cu") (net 1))
 (segment (start 160.02 95.82) (end 160.02 104.14) (width 0.6) (layer "F.Cu") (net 1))
 (segment (start 164.4 91.44) (end 169.32 86.52) (width 0.6) (layer "F.Cu") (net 1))
 (segment (start 73.66 58.42) (end 96.52 58.42) (width 0.6) (layer "F.Cu") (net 1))
 (segment (start 99.06 91.44) (end 93.98 91.44) (width 0.6) (layer "F.Cu") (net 1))
 (segment (start 96.52 58.42) (end 101.6 53.34) (width 0.6) (layer "F.Cu") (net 1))
 (segment (start 81.28 73.66) (end 73.66 66.04) (width 0.6) (layer "F.Cu") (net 1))
 (segment (start 137.12 45.68) (end 139.7 48.26) (width 0.6) (layer "F.Cu") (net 1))
 (segment (start 139.62 78.74) (end 139.7 78.74) (width 0.6) (layer "F.Cu") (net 1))
 (segment (start 73.66 66.04) (end 73.66 58.42) (width 0.6) (layer "F.Cu") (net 1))
 (segment (start 164.4 91.44) (end 160.02 95.82) (width 0.6) (layer "F.Cu") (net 1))
 (segment (start 115.951 49.784) (end 125.476 49.784) (width 0.6) (layer "F.Cu") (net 1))
 (segment (start 164.4 91.44) (end 152.4 91.44) (width 0.6) (layer "F.Cu") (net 1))
 (segment (start 160.02 104.14) (end 163.83 107.95) (width 0.6) (layer "F.Cu") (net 1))
 (segment (start 132.08 71.2) (end 114.3 53.42) (width 0.6) (layer "F.Cu") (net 1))
 (segment (start 172.72 68.58) (end 180.34 68.58) (width 0.6) (layer "F.Cu") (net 1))
 (segment (start 154.94 121.92) (end 163.83 121.92) (width 0.6) (layer "F.Cu") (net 1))
 (segment (start 93.98 91.44) (end 93.98 104.14) (width 0.6) (layer "F.Cu") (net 1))
 (segment (start 163.83 107.95) (end 163.83 121.92) (width 0.6) (layer "F.Cu") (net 1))
 (segment (start 139.7 118.11) (end 152.4 118.11) (width 0.6) (layer "F.Cu") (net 1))
 (segment (start 106.59 73.66) (end 109.72 76.79) (width 0.6) (layer "F.Cu") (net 1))
 (segment (start 114.3 53.34) (end 115.951 51.689) (width 0.6) (layer "F.Cu") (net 1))
 (segment (start 114.3 53.42) (end 114.3 53.34) (width 0.6) (layer "F.Cu") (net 1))
 (segment (start 182.88 71.12) (end 180.34 73.66) (width 0.6) (layer "F.Cu") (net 1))
 (segment (start 102.19 102.19) (end 99.06 99.06) (width 0.6) (layer "F.Cu") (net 16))
 (segment (start 109.72 102.19) (end 102.19 102.19) (width 0.6) (layer "F.Cu") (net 16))
 (segment (start 109.13 96.52) (end 109.72 97.11) (width 0.6) (layer "F.Cu") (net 14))
 (segment (start 99.06 96.52) (end 109.13 96.52) (width 0.6) (layer "F.Cu") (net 14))
 (segment (start 111.76 106.68) (end 111.76 101.69) (width 0.6) (layer "F.Cu") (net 15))
 (segment (start 101.6 109.22) (end 109.22 109.22) (width 0.6) (layer "F.Cu") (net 15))
 (segment (start 96.52 104.14) (end 101.6 109.22) (width 0.6) (layer "F.Cu") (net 15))
 (segment (start 111.76 101.69) (end 109.72 99.65) (width 0.6) (layer "F.Cu") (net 15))
 (segment (start 99.06 93.98) (end 96.52 96.52) (width 0.6) (layer "F.Cu") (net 15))
 (segment (start 96.52 96.52) (end 96.52 104.14) (width 0.6) (layer "F.Cu") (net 15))
 (segment (start 109.22 109.22) (end 111.76 106.68) (width 0.6) (layer "F.Cu") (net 15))
 (segment (start 139.11 84.41) (end 139.7 83.82) (width 0.6) (layer "F.Cu") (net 25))
 (segment (start 124.96 84.41) (end 139.11 84.41) (width 0.6) (layer "F.Cu") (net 25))
 (segment (start 139.7 83.82) (end 152.4 96.52) (width 0.6) (layer "F.Cu") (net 25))
 (segment (start 124.96 86.95) (end 139.11 86.95) (width 0.6) (layer "F.Cu") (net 24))
 (segment (start 139.7 86.36) (end 152.4 99.06) (width 0.6) (layer "F.Cu") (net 24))
 (segment (start 139.11 86.95) (end 139.7 86.36) (width 0.6) (layer "F.Cu") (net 24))
 (segment (start 124.96 97.11) (end 130.13 97.11) (width 0.6) (layer "F.Cu") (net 21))
 (segment (start 130.13 97.11) (end 144.78 111.76) (width 0.6) (layer "F.Cu") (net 21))
 (segment (start 139.7 110.49) (end 143.51 110.49) (width 0.6) (layer "F.Cu") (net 21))
 (segment (start 143.51 110.49) (end 144.78 111.76) (width 0.6) (layer "F.Cu") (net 21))
 (segment (start 152.4 110.49) (end 156.21 110.49) (width 0.6) (layer "F.Cu") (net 3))
 (segment (start 156.21 110.49) (end 157.48 111.76) (width 0.6) (layer "F.Cu") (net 3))
 (segment (start 140.29 94.57) (end 157.48 111.76) (width 0.6) (layer "F.Cu") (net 3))
 (segment (start 124.96 94.57) (end 140.29 94.57) (width 0.6) (layer "F.Cu") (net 3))
 (segment (start 93.345 40.64) (end 97.409 36.576) (width 0.6) (layer "F.Cu") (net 37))
 (segment (start 82.2 40.64) (end 93.345 40.64) (width 0.6) (layer "F.Cu") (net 37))
 (segment (start 76.2 40.64) (end 78.65 43.09) (width 0.6) (layer "F.Cu") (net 38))
 (segment (start 90.715 43.09) (end 97.409 49.784) (width 0.6) (layer "F.Cu") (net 38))
 (segment (start 78.65 43.09) (end 90.715 43.09) (width 0.6) (layer "F.Cu") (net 38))
 (segment (start 172.72 88.9) (end 167.64 93.98) (width 0.6) (layer "F.Cu") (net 34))
 (segment (start 167.64 93.98) (end 164.4 93.98) (width 0.6) (layer "F.Cu") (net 34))
 (segment (start 177.8 71.12) (end 172.72 76.2) (width 0.6) (layer "F.Cu") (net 34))
 (segment (start 172.72 76.2) (end 172.72 88.9) (width 0.6) (layer "F.Cu") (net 34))
 (segment (start 172.02 104.14) (end 177.8 104.14) (width 0.6) (layer "F.Cu") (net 35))
 (segment (start 164.4 96.52) (end 172.02 104.14) (width 0.6) (layer "F.Cu") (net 35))
 (segment (start 182.88 109.22) (end 187.96 104.14) (width 0.6) (layer "F.Cu") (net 36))
 (segment (start 187.96 104.14) (end 187.96 99.06) (width 0.6) (layer "F.Cu") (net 36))
 (segment (start 187.96 99.06) (end 185.42 96.52) (width 0.6) (layer "F.Cu") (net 36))
 (segment (start 185.42 96.52) (end 177.8 96.52) (width 0.6) (layer "F.Cu") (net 36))
 (segment (start 164.4 99.06) (end 174.56 109.22) (width 0.6) (layer "F.Cu") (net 36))
 (segment (start 174.56 109.22) (end 182.88 109.22) (width 0.6) (layer "F.Cu") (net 36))
 (segment (start 114.3 68.58) (end 114.3 78.74) (width 0.6) (layer "F.Cu") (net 9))
 (segment (start 111.17 81.87) (end 109.72 81.87) (width 0.6) (layer "F.Cu") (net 9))
 (segment (start 102.31 67.87) (end 106.68 63.5) (width 0.6) (layer "F.Cu") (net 9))
 (segment (start 106.68 63.5) (end 109.22 63.5) (width 0.6) (layer "F.Cu") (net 9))
 (segment (start 93.98 68.58) (end 94.69 67.87) (width 0.6) (layer "F.Cu") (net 9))
 (segment (start 114.3 78.74) (end 111.17 81.87) (width 0.6) (layer "F.Cu") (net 9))
 (segment (start 109.22 63.5) (end 114.3 68.58) (width 0.6) (layer "F.Cu") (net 9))
 (segment (start 94.69 67.87) (end 102.31 67.87) (width 0.6) (layer "F.Cu") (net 9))
 (segment (start 81.28 68.58) (end 81.28 69.77) (width 0.6) (layer "F.Cu") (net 4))
 (segment (start 92.03 89.49) (end 109.72 89.49) (width 0.6) (layer "F.Cu") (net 4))
 (segment (start 92.03 79.960811) (end 92.03 89.49) (width 0.6) (layer "F.Cu") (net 4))
 (segment (start 81.839189 69.77) (end 92.03 79.960811) (width 0.6) (layer "F.Cu") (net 4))
 (segment (start 81.28 69.77) (end 81.839189 69.77) (width 0.6) (layer "F.Cu") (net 4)))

